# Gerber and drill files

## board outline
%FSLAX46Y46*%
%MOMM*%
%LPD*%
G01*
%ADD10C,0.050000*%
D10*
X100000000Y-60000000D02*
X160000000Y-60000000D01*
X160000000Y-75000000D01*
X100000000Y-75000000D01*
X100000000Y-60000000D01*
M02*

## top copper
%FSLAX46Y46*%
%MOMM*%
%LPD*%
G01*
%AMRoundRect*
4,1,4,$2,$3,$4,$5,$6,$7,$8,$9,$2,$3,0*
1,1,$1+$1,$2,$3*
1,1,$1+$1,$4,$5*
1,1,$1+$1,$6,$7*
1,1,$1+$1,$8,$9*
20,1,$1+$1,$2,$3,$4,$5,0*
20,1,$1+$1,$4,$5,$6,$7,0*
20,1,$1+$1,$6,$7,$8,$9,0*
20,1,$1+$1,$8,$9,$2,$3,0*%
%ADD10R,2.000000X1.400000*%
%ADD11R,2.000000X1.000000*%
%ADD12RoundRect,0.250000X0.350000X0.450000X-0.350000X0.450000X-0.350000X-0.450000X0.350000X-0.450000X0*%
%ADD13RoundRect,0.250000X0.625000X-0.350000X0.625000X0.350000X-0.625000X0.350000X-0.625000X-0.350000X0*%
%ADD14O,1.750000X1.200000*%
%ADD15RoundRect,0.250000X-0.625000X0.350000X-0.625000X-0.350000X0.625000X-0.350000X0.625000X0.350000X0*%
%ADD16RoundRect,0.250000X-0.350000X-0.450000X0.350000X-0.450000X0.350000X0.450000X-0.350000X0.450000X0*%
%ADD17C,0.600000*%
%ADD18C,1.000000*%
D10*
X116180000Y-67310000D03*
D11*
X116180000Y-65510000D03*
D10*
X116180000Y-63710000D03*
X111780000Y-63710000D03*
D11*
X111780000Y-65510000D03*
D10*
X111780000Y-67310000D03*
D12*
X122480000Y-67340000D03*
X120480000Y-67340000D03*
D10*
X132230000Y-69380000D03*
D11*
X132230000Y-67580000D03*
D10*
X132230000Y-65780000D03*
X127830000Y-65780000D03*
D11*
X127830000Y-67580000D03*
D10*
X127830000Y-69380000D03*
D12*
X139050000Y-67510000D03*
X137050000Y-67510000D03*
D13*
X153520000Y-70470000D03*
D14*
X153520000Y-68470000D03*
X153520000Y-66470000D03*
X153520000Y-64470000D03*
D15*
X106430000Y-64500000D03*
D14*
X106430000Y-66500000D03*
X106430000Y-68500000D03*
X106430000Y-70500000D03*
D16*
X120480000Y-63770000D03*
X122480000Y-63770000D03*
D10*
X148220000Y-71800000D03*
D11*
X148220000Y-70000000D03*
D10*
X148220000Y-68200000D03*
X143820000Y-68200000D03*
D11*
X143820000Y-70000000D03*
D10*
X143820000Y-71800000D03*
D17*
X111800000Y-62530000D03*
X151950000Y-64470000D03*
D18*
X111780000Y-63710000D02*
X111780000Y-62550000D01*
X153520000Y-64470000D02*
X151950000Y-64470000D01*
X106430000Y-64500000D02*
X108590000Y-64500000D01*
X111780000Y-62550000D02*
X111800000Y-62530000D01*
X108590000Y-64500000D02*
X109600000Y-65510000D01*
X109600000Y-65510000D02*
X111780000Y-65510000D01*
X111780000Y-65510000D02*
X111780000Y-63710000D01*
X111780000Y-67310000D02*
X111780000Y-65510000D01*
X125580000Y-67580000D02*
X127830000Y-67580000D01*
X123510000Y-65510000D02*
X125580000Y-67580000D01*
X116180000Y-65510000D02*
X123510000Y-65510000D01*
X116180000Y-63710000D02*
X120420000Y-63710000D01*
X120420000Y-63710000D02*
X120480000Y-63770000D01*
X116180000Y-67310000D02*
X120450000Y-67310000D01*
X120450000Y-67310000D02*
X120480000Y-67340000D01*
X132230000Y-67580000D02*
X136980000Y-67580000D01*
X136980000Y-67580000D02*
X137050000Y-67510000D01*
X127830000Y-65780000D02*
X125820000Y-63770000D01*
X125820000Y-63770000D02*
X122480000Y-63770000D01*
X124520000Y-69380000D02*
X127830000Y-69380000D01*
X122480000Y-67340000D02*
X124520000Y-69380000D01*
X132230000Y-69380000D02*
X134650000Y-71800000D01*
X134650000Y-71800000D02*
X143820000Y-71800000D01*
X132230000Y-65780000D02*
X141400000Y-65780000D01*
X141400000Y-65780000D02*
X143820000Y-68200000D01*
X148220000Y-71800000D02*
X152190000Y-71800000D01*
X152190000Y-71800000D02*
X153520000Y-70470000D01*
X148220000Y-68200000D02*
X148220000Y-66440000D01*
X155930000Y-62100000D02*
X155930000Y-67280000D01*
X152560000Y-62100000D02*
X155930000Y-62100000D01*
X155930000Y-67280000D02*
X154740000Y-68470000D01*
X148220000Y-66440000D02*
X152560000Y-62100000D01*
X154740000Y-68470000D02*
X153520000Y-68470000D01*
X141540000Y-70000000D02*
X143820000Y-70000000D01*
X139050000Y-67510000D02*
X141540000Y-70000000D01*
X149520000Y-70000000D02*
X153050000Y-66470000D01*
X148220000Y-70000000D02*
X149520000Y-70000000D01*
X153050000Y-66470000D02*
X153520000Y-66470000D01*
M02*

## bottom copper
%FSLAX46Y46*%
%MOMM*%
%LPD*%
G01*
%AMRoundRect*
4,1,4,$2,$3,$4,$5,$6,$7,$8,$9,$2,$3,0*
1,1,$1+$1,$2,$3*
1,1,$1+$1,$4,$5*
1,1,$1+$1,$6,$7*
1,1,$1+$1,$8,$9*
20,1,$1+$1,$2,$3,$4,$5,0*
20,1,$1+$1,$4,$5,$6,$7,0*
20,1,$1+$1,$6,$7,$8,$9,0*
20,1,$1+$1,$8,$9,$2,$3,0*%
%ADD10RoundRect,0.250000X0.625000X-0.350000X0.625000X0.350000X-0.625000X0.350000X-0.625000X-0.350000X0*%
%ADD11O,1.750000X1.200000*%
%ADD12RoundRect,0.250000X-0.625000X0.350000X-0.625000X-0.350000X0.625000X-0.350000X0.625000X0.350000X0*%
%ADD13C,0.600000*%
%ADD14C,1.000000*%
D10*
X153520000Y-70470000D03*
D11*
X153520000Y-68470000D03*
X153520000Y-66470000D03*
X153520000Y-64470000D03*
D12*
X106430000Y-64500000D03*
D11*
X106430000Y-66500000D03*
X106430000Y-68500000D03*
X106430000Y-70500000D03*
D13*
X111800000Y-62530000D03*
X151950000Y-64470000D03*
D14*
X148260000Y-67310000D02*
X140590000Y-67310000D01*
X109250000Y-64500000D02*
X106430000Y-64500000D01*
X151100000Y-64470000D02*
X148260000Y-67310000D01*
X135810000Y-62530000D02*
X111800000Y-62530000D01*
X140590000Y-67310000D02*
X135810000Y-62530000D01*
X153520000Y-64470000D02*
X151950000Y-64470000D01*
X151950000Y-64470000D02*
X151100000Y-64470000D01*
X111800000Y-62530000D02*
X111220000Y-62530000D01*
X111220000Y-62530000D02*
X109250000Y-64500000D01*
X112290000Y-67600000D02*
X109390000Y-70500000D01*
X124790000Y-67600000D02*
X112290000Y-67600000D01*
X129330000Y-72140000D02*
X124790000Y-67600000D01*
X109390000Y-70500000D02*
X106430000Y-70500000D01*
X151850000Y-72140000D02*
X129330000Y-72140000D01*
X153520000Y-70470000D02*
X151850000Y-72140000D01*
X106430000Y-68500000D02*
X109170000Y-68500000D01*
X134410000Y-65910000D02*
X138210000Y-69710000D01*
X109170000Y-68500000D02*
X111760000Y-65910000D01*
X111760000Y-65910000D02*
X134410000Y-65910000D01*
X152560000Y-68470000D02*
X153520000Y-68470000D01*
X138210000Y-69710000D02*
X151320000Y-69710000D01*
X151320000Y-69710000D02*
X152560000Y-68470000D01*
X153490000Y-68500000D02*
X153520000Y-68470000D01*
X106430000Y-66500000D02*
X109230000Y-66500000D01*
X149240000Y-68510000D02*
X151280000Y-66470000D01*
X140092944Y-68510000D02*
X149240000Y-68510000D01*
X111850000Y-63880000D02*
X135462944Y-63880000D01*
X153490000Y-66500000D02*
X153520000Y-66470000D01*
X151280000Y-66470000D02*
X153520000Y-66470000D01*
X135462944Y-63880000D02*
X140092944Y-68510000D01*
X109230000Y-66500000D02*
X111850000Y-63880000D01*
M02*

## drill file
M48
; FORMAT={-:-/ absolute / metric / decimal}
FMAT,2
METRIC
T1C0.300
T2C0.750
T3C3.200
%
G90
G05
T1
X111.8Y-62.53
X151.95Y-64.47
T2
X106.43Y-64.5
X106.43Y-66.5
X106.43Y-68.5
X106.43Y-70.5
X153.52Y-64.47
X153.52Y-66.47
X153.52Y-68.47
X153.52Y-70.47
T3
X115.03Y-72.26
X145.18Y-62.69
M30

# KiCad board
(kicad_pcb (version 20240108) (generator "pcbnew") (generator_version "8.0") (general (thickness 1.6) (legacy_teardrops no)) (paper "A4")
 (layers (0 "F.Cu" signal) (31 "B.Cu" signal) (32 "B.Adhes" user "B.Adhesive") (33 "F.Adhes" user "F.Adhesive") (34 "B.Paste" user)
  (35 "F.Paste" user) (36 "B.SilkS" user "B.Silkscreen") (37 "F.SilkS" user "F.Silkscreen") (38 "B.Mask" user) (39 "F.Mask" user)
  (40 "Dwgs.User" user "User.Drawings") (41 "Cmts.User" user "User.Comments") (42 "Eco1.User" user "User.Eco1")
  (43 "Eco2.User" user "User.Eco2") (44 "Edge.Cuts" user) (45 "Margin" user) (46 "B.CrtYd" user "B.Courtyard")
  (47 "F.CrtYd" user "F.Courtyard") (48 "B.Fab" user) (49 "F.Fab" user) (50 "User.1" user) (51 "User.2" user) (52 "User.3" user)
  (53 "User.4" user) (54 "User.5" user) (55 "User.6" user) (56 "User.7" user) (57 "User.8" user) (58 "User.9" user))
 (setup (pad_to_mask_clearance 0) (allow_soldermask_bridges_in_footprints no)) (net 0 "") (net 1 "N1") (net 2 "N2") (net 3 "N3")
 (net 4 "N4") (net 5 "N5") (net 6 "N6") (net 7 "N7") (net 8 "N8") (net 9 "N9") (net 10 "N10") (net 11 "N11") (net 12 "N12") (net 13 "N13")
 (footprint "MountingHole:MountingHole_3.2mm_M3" (layer "F.Cu") (at 115.03 72.26)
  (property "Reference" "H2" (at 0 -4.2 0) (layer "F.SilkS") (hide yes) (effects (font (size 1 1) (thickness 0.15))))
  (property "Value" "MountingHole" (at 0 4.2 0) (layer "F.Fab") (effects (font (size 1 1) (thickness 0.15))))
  (pad "" np_thru_hole circle (at 0 0) (size 3.2 3.2) (drill 3.2) (layers "F&B.Cu")))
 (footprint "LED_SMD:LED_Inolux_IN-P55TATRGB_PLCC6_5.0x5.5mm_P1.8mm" (layer "F.Cu") (at 113.98 65.51 180)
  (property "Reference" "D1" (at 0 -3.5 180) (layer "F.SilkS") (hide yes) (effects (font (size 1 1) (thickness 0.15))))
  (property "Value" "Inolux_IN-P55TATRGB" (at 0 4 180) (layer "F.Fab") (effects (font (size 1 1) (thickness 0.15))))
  (pad "1" smd rect (at -2.2 -1.8 180) (size 2 1.4) (layers "F.Cu" "F.Paste" "F.Mask") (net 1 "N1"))
  (pad "2" smd rect (at -2.2 0 180) (size 2 1) (layers "F.Cu" "F.Paste" "F.Mask") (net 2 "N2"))
  (pad "3" smd rect (at -2.2 1.8 180) (size 2 1.4) (layers "F.Cu" "F.Paste" "F.Mask") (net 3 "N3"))
  (pad "4" smd rect (at 2.2 1.8 180) (size 2 1.4) (layers "F.Cu" "F.Paste" "F.Mask") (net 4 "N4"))
  (pad "5" smd rect (at 2.2 0 180) (size 2 1) (layers "F.Cu" "F.Paste" "F.Mask") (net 4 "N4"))
  (pad "6" smd rect (at 2.2 -1.8 180) (size 2 1.4) (layers "F.Cu" "F.Paste" "F.Mask") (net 4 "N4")))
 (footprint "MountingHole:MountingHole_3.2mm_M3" (layer "F.Cu") (at 145.18 62.69)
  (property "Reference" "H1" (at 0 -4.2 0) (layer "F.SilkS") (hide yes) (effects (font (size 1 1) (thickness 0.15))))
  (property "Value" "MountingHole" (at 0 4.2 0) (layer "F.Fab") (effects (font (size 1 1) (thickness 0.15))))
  (pad "" np_thru_hole circle (at 0 0) (size 3.2 3.2) (drill 3.2) (layers "F&B.Cu" "B.Mask")))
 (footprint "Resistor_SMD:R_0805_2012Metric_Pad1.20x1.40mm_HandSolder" (layer "F.Cu") (at 121.48 67.34 180)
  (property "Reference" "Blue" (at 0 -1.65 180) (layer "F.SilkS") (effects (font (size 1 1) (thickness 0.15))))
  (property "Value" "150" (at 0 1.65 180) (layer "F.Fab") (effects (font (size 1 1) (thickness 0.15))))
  (pad "1" smd roundrect (at -1 0 180) (size 1.2 1.4) (layers "F.Cu" "F.Paste" "F.Mask") (roundrect_rratio 0.208333) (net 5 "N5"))
  (pad "2" smd roundrect (at 1 0 180) (size 1.2 1.4) (layers "F.Cu" "F.Paste" "F.Mask") (roundrect_rratio 0.208333) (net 1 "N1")))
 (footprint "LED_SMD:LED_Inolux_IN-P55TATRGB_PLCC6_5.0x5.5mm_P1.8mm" (layer "F.Cu") (at 130.03 67.58 180)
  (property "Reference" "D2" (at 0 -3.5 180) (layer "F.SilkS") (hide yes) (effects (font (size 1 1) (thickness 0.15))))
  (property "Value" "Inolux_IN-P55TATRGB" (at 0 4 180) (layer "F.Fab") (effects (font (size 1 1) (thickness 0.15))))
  (pad "1" smd rect (at -2.2 -1.8 180) (size 2 1.4) (layers "F.Cu" "F.Paste" "F.Mask") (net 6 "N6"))
  (pad "2" smd rect (at -2.2 0 180) (size 2 1) (layers "F.Cu" "F.Paste" "F.Mask") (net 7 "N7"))
  (pad "3" smd rect (at -2.2 1.8 180) (size 2 1.4) (layers "F.Cu" "F.Paste" "F.Mask") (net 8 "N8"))
  (pad "4" smd rect (at 2.2 1.8 180) (size 2 1.4) (layers "F.Cu" "F.Paste" "F.Mask") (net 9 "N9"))
  (pad "5" smd rect (at 2.2 0 180) (size 2 1) (layers "F.Cu" "F.Paste" "F.Mask") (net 2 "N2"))
  (pad "6" smd rect (at 2.2 -1.8 180) (size 2 1.4) (layers "F.Cu" "F.Paste" "F.Mask") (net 5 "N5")))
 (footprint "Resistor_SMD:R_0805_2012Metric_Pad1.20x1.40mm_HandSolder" (layer "F.Cu") (at 138.05 67.51 180)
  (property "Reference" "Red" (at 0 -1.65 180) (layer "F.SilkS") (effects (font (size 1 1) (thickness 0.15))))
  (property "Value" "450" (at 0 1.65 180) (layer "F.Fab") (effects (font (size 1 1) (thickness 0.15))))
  (pad "1" smd roundrect (at -1 0 180) (size 1.2 1.4) (layers "F.Cu" "F.Paste" "F.Mask") (roundrect_rratio 0.208333) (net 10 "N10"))
  (pad "2" smd roundrect (at 1 0 180) (size 1.2 1.4) (layers "F.Cu" "F.Paste" "F.Mask") (roundrect_rratio 0.208333) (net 7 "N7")))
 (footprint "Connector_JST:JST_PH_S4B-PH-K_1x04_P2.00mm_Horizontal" (layer "F.Cu") (at 153.52 70.47 90)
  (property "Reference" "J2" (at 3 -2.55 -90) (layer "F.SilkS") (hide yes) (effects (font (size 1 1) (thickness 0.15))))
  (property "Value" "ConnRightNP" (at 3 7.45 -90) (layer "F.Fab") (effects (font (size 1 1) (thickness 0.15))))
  (pad "1" thru_hole roundrect (at 0 0 90) (size 1.2 1.75) (drill 0.75) (layers "*.Cu" "*.Mask") (remove_unused_layers no)
   (roundrect_rratio 0.208333) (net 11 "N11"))
  (pad "2" thru_hole oval (at 2 0 90) (size 1.2 1.75) (drill 0.75) (layers "*.Cu" "*.Mask") (remove_unused_layers no) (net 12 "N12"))
  (pad "3" thru_hole oval (at 4 0 90) (size 1.2 1.75) (drill 0.75) (layers "*.Cu" "*.Mask") (remove_unused_layers no) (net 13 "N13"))
  (pad "4" thru_hole oval (at 6 0 90) (size 1.2 1.75) (drill 0.75) (layers "*.Cu" "*.Mask") (remove_unused_layers no) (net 4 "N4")))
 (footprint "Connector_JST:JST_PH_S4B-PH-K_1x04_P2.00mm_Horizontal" (layer "F.Cu") (at 106.43 64.5 -90)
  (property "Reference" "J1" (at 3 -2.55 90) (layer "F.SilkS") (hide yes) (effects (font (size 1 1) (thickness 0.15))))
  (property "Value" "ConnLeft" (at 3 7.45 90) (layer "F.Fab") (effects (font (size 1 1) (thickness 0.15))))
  (pad "1" thru_hole roundrect (at 0 0 270) (size 1.2 1.75) (drill 0.75) (layers "*.Cu" "*.Mask") (remove_unused_layers no)
   (roundrect_rratio 0.208333) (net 4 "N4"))
  (pad "2" thru_hole oval (at 2 0 270) (size 1.2 1.75) (drill 0.75) (layers "*.Cu" "*.Mask") (remove_unused_layers no) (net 13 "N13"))
  (pad "3" thru_hole oval (at 4 0 270) (size 1.2 1.75) (drill 0.75) (layers "*.Cu" "*.Mask") (remove_unused_layers no) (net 12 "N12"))
  (pad "4" thru_hole oval (at 6 0 270) (size 1.2 1.75) (drill 0.75) (layers "*.Cu" "*.Mask") (remove_unused_layers no) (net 11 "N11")))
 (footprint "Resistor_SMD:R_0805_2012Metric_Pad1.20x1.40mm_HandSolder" (layer "F.Cu") (at 121.48 63.77)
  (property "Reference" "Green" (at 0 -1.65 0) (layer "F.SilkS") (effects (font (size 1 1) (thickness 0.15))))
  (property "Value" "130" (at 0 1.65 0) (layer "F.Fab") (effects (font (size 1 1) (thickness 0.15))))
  (pad "1" smd roundrect (at -1 0) (size 1.2 1.4) (layers "F.Cu" "F.Paste" "F.Mask") (roundrect_rratio 0.208333) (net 3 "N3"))
  (pad "2" smd roundrect (at 1 0) (size 1.2 1.4) (layers "F.Cu" "F.Paste" "F.Mask") (roundrect_rratio 0.208333) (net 9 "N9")))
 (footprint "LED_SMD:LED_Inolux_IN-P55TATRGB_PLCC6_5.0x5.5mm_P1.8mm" (layer "F.Cu") (at 146.02 70 180)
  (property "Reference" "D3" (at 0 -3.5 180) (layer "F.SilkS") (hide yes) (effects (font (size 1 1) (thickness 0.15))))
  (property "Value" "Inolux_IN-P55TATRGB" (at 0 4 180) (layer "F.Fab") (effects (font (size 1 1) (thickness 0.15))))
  (pad "1" smd rect (at -2.2 -1.8 180) (size 2 1.4) (layers "F.Cu" "F.Paste" "F.Mask") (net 11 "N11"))
  (pad "2" smd rect (at -2.2 0 180) (size 2 1) (layers "F.Cu" "F.Paste" "F.Mask") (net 13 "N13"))
  (pad "3" smd rect (at -2.2 1.8 180) (size 2 1.4) (layers "F.Cu" "F.Paste" "F.Mask") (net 12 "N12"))
  (pad "4" smd rect (at 2.2 1.8 180) (size 2 1.4) (layers "F.Cu" "F.Paste" "F.Mask") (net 8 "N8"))
  (pad "5" smd rect (at 2.2 0 180) (size 2 1) (layers "F.Cu" "F.Paste" "F.Mask") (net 10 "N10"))
  (pad "6" smd rect (at 2.2 -1.8 180) (size 2 1.4) (layers "F.Cu" "F.Paste" "F.Mask") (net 6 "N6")))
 (gr_rect (start 100 60) (end 160 75) (stroke (width 0.05) (type default)) (fill none) (layer "Edge.Cuts"))
 (segment (start 111.78 63.71) (end 111.78 62.55) (width 1) (layer "F.Cu") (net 4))
 (segment (start 153.52 64.47) (end 151.95 64.47) (width 1) (layer "F.Cu") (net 4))
 (segment (start 106.43 64.5) (end 108.59 64.5) (width 1) (layer "F.Cu") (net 4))
 (segment (start 111.78 62.55) (end 111.8 62.53) (width 1) (layer "F.Cu") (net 4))
 (segment (start 108.59 64.5) (end 109.6 65.51) (width 1) (layer "F.Cu") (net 4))
 (segment (start 109.6 65.51) (end 111.78 65.51) (width 1) (layer "F.Cu") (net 4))
 (segment (start 111.78 65.51) (end 111.78 63.71) (width 1) (layer "F.Cu") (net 4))
 (segment (start 111.78 67.31) (end 111.78 65.51) (width 1) (layer "F.Cu") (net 4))
 (via (at 111.8 62.53) (size 0.6) (drill 0.3) (layers "F.Cu" "B.Cu") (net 4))
 (via (at 151.95 64.47) (size 0.6) (drill 0.3) (layers "F.Cu" "B.Cu") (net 4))
 (segment (start 148.26 67.31) (end 140.59 67.31) (width 1) (layer "B.Cu") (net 4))
 (segment (start 109.25 64.5) (end 106.43 64.5) (width 1) (layer "B.Cu") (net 4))
 (segment (start 151.1 64.47) (end 148.26 67.31) (width 1) (layer "B.Cu") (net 4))
 (segment (start 135.81 62.53) (end 111.8 62.53) (width 1) (layer "B.Cu") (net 4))
 (segment (start 140.59 67.31) (end 135.81 62.53) (width 1) (layer "B.Cu") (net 4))
 (segment (start 153.52 64.47) (end 151.95 64.47) (width 1) (layer "B.Cu") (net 4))
 (segment (start 151.95 64.47) (end 151.1 64.47) (width 1) (layer "B.Cu") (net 4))
 (segment (start 111.8 62.53) (end 111.22 62.53) (width 1) (layer "B.Cu") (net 4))
 (segment (start 111.22 62.53) (end 109.25 64.5) (width 1) (layer "B.Cu") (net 4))
 (segment (start 125.58 67.58) (end 127.83 67.58) (width 1) (layer "F.Cu") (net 2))
 (segment (start 123.51 65.51) (end 125.58 67.58) (width 1) (layer "F.Cu") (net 2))
 (segment (start 116.18 65.51) (end 123.51 65.51) (width 1) (layer "F.Cu") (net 2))
 (segment (start 116.18 63.71) (end 120.42 63.71) (width 1) (layer "F.Cu") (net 3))
 (segment (start 120.42 63.71) (end 120.48 63.77) (width 1) (layer "F.Cu") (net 3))
 (segment (start 116.18 67.31) (end 120.45 67.31) (width 1) (layer "F.Cu") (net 1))
 (segment (start 120.45 67.31) (end 120.48 67.34) (width 1) (layer "F.Cu") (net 1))
 (segment (start 132.23 67.58) (end 136.98 67.58) (width 1) (layer "F.Cu") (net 7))
 (segment (start 136.98 67.58) (end 137.05 67.51) (width 1) (layer "F.Cu") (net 7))
 (segment (start 127.83 65.78) (end 125.82 63.77) (width 1) (layer "F.Cu") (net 9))
 (segment (start 125.82 63.77) (end 122.48 63.77) (width 1) (layer "F.Cu") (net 9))
 (segment (start 124.52 69.38) (end 127.83 69.38) (width 1) (layer "F.Cu") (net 5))
 (segment (start 122.48 67.34) (end 124.52 69.38) (width 1) (layer "F.Cu") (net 5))
 (segment (start 132.23 69.38) (end 134.65 71.8) (width 1) (layer "F.Cu") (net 6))
 (segment (start 134.65 71.8) (end 143.82 71.8) (width 1) (layer "F.Cu") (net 6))
 (segment (start 132.23 65.78) (end 141.4 65.78) (width 1) (layer "F.Cu") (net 8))
 (segment (start 141.4 65.78) (end 143.82 68.2) (width 1) (layer "F.Cu") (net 8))
 (segment (start 148.22 71.8) (end 152.19 71.8) (width 1) (layer "F.Cu") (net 11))
 (segment (start 152.19 71.8) (end 153.52 70.47) (width 1) (layer "F.Cu") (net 11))
 (segment (start 112.29 67.6) (end 109.39 70.5) (width 1) (layer "B.Cu") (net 11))
 (segment (start 124.79 67.6) (end 112.29 67.6) (width 1) (layer "B.Cu") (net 11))
 (segment (start 129.33 72.14) (end 124.79 67.6) (width 1) (layer "B.Cu") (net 11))
 (segment (start 109.39 70.5) (end 106.43 70.5) (width 1) (layer "B.Cu") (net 11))
 (segment (start 151.85 72.14) (end 129.33 72.14) (width 1) (layer "B.Cu") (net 11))
 (segment (start 153.52 70.47) (end 151.85 72.14) (width 1) (layer "B.Cu") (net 11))
 (segment (start 148.22 68.2) (end 148.22 66.44) (width 1) (layer "F.Cu") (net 12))
 (segment (start 155.93 62.1) (end 155.93 67.28) (width 1) (layer "F.Cu") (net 12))
 (segment (start 152.56 62.1) (end 155.93 62.1) (width 1) (layer "F.Cu") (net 12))
 (segment (start 155.93 67.28) (end 154.74 68.47) (width 1) (layer "F.Cu") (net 12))
 (segment (start 148.22 66.44) (end 152.56 62.1) (width 1) (layer "F.Cu") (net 12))
 (segment (start 154.74 68.47) (end 153.52 68.47) (width 1) (layer "F.Cu") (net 12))
 (segment (start 106.43 68.5) (end 109.17 68.5) (width 1) (layer "B.Cu") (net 12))
 (segment (start 134.41 65.91) (end 138.21 69.71) (width 1) (layer "B.Cu") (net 12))
 (segment (start 109.17 68.5) (end 111.76 65.91) (width 1) (layer "B.Cu") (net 12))
 (segment (start 111.76 65.91) (end 134.41 65.91) (width 1) (layer "B.Cu") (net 12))
 (segment (start 152.56 68.47) (end 153.52 68.47) (width 1) (layer "B.Cu") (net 12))
 (segment (start 138.21 69.71) (end 151.32 69.71) (width 1) (layer "B.Cu") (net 12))
 (segment (start 151.32 69.71) (end 152.56 68.47) (width 1) (layer "B.Cu") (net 12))
 (segment (start 153.49 68.5) (end 153.52 68.47) (width 1) (layer "B.Cu") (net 12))
 (segment (start 141.54 70) (end 143.82 70) (width 1) (layer "F.Cu") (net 10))
 (segment (start 139.05 67.51) (end 141.54 70) (width 1) (layer "F.Cu") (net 10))
 (segment (start 149.52 70) (end 153.05 66.47) (width 1) (layer "F.Cu") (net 13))
 (segment (start 148.22 70) (end 149.52 70) (width 1) (layer "F.Cu") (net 13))
 (segment (start 153.05 66.47) (end 153.52 66.47) (width 1) (layer "F.Cu") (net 13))
 (segment (start 106.43 66.5) (end 109.23 66.5) (width 1) (layer "B.Cu") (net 13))
 (segment (start 149.24 68.51) (end 151.28 66.47) (width 1) (layer "B.Cu") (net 13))
 (segment (start 140.092944 68.51) (end 149.24 68.51) (width 1) (layer "B.Cu") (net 13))
 (segment (start 111.85 63.88) (end 135.462944 63.88) (width 1) (layer "B.Cu") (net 13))
 (segment (start 153.49 66.5) (end 153.52 66.47) (width 1) (layer "B.Cu") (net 13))
 (segment (start 151.28 66.47) (end 153.52 66.47) (width 1) (layer "B.Cu") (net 13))
 (segment (start 135.462944 63.88) (end 140.092944 68.51) (width 1) (layer "B.Cu") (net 13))
 (segment (start 109.23 66.5) (end 111.85 63.88) (width 1) (layer "B.Cu") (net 13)))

